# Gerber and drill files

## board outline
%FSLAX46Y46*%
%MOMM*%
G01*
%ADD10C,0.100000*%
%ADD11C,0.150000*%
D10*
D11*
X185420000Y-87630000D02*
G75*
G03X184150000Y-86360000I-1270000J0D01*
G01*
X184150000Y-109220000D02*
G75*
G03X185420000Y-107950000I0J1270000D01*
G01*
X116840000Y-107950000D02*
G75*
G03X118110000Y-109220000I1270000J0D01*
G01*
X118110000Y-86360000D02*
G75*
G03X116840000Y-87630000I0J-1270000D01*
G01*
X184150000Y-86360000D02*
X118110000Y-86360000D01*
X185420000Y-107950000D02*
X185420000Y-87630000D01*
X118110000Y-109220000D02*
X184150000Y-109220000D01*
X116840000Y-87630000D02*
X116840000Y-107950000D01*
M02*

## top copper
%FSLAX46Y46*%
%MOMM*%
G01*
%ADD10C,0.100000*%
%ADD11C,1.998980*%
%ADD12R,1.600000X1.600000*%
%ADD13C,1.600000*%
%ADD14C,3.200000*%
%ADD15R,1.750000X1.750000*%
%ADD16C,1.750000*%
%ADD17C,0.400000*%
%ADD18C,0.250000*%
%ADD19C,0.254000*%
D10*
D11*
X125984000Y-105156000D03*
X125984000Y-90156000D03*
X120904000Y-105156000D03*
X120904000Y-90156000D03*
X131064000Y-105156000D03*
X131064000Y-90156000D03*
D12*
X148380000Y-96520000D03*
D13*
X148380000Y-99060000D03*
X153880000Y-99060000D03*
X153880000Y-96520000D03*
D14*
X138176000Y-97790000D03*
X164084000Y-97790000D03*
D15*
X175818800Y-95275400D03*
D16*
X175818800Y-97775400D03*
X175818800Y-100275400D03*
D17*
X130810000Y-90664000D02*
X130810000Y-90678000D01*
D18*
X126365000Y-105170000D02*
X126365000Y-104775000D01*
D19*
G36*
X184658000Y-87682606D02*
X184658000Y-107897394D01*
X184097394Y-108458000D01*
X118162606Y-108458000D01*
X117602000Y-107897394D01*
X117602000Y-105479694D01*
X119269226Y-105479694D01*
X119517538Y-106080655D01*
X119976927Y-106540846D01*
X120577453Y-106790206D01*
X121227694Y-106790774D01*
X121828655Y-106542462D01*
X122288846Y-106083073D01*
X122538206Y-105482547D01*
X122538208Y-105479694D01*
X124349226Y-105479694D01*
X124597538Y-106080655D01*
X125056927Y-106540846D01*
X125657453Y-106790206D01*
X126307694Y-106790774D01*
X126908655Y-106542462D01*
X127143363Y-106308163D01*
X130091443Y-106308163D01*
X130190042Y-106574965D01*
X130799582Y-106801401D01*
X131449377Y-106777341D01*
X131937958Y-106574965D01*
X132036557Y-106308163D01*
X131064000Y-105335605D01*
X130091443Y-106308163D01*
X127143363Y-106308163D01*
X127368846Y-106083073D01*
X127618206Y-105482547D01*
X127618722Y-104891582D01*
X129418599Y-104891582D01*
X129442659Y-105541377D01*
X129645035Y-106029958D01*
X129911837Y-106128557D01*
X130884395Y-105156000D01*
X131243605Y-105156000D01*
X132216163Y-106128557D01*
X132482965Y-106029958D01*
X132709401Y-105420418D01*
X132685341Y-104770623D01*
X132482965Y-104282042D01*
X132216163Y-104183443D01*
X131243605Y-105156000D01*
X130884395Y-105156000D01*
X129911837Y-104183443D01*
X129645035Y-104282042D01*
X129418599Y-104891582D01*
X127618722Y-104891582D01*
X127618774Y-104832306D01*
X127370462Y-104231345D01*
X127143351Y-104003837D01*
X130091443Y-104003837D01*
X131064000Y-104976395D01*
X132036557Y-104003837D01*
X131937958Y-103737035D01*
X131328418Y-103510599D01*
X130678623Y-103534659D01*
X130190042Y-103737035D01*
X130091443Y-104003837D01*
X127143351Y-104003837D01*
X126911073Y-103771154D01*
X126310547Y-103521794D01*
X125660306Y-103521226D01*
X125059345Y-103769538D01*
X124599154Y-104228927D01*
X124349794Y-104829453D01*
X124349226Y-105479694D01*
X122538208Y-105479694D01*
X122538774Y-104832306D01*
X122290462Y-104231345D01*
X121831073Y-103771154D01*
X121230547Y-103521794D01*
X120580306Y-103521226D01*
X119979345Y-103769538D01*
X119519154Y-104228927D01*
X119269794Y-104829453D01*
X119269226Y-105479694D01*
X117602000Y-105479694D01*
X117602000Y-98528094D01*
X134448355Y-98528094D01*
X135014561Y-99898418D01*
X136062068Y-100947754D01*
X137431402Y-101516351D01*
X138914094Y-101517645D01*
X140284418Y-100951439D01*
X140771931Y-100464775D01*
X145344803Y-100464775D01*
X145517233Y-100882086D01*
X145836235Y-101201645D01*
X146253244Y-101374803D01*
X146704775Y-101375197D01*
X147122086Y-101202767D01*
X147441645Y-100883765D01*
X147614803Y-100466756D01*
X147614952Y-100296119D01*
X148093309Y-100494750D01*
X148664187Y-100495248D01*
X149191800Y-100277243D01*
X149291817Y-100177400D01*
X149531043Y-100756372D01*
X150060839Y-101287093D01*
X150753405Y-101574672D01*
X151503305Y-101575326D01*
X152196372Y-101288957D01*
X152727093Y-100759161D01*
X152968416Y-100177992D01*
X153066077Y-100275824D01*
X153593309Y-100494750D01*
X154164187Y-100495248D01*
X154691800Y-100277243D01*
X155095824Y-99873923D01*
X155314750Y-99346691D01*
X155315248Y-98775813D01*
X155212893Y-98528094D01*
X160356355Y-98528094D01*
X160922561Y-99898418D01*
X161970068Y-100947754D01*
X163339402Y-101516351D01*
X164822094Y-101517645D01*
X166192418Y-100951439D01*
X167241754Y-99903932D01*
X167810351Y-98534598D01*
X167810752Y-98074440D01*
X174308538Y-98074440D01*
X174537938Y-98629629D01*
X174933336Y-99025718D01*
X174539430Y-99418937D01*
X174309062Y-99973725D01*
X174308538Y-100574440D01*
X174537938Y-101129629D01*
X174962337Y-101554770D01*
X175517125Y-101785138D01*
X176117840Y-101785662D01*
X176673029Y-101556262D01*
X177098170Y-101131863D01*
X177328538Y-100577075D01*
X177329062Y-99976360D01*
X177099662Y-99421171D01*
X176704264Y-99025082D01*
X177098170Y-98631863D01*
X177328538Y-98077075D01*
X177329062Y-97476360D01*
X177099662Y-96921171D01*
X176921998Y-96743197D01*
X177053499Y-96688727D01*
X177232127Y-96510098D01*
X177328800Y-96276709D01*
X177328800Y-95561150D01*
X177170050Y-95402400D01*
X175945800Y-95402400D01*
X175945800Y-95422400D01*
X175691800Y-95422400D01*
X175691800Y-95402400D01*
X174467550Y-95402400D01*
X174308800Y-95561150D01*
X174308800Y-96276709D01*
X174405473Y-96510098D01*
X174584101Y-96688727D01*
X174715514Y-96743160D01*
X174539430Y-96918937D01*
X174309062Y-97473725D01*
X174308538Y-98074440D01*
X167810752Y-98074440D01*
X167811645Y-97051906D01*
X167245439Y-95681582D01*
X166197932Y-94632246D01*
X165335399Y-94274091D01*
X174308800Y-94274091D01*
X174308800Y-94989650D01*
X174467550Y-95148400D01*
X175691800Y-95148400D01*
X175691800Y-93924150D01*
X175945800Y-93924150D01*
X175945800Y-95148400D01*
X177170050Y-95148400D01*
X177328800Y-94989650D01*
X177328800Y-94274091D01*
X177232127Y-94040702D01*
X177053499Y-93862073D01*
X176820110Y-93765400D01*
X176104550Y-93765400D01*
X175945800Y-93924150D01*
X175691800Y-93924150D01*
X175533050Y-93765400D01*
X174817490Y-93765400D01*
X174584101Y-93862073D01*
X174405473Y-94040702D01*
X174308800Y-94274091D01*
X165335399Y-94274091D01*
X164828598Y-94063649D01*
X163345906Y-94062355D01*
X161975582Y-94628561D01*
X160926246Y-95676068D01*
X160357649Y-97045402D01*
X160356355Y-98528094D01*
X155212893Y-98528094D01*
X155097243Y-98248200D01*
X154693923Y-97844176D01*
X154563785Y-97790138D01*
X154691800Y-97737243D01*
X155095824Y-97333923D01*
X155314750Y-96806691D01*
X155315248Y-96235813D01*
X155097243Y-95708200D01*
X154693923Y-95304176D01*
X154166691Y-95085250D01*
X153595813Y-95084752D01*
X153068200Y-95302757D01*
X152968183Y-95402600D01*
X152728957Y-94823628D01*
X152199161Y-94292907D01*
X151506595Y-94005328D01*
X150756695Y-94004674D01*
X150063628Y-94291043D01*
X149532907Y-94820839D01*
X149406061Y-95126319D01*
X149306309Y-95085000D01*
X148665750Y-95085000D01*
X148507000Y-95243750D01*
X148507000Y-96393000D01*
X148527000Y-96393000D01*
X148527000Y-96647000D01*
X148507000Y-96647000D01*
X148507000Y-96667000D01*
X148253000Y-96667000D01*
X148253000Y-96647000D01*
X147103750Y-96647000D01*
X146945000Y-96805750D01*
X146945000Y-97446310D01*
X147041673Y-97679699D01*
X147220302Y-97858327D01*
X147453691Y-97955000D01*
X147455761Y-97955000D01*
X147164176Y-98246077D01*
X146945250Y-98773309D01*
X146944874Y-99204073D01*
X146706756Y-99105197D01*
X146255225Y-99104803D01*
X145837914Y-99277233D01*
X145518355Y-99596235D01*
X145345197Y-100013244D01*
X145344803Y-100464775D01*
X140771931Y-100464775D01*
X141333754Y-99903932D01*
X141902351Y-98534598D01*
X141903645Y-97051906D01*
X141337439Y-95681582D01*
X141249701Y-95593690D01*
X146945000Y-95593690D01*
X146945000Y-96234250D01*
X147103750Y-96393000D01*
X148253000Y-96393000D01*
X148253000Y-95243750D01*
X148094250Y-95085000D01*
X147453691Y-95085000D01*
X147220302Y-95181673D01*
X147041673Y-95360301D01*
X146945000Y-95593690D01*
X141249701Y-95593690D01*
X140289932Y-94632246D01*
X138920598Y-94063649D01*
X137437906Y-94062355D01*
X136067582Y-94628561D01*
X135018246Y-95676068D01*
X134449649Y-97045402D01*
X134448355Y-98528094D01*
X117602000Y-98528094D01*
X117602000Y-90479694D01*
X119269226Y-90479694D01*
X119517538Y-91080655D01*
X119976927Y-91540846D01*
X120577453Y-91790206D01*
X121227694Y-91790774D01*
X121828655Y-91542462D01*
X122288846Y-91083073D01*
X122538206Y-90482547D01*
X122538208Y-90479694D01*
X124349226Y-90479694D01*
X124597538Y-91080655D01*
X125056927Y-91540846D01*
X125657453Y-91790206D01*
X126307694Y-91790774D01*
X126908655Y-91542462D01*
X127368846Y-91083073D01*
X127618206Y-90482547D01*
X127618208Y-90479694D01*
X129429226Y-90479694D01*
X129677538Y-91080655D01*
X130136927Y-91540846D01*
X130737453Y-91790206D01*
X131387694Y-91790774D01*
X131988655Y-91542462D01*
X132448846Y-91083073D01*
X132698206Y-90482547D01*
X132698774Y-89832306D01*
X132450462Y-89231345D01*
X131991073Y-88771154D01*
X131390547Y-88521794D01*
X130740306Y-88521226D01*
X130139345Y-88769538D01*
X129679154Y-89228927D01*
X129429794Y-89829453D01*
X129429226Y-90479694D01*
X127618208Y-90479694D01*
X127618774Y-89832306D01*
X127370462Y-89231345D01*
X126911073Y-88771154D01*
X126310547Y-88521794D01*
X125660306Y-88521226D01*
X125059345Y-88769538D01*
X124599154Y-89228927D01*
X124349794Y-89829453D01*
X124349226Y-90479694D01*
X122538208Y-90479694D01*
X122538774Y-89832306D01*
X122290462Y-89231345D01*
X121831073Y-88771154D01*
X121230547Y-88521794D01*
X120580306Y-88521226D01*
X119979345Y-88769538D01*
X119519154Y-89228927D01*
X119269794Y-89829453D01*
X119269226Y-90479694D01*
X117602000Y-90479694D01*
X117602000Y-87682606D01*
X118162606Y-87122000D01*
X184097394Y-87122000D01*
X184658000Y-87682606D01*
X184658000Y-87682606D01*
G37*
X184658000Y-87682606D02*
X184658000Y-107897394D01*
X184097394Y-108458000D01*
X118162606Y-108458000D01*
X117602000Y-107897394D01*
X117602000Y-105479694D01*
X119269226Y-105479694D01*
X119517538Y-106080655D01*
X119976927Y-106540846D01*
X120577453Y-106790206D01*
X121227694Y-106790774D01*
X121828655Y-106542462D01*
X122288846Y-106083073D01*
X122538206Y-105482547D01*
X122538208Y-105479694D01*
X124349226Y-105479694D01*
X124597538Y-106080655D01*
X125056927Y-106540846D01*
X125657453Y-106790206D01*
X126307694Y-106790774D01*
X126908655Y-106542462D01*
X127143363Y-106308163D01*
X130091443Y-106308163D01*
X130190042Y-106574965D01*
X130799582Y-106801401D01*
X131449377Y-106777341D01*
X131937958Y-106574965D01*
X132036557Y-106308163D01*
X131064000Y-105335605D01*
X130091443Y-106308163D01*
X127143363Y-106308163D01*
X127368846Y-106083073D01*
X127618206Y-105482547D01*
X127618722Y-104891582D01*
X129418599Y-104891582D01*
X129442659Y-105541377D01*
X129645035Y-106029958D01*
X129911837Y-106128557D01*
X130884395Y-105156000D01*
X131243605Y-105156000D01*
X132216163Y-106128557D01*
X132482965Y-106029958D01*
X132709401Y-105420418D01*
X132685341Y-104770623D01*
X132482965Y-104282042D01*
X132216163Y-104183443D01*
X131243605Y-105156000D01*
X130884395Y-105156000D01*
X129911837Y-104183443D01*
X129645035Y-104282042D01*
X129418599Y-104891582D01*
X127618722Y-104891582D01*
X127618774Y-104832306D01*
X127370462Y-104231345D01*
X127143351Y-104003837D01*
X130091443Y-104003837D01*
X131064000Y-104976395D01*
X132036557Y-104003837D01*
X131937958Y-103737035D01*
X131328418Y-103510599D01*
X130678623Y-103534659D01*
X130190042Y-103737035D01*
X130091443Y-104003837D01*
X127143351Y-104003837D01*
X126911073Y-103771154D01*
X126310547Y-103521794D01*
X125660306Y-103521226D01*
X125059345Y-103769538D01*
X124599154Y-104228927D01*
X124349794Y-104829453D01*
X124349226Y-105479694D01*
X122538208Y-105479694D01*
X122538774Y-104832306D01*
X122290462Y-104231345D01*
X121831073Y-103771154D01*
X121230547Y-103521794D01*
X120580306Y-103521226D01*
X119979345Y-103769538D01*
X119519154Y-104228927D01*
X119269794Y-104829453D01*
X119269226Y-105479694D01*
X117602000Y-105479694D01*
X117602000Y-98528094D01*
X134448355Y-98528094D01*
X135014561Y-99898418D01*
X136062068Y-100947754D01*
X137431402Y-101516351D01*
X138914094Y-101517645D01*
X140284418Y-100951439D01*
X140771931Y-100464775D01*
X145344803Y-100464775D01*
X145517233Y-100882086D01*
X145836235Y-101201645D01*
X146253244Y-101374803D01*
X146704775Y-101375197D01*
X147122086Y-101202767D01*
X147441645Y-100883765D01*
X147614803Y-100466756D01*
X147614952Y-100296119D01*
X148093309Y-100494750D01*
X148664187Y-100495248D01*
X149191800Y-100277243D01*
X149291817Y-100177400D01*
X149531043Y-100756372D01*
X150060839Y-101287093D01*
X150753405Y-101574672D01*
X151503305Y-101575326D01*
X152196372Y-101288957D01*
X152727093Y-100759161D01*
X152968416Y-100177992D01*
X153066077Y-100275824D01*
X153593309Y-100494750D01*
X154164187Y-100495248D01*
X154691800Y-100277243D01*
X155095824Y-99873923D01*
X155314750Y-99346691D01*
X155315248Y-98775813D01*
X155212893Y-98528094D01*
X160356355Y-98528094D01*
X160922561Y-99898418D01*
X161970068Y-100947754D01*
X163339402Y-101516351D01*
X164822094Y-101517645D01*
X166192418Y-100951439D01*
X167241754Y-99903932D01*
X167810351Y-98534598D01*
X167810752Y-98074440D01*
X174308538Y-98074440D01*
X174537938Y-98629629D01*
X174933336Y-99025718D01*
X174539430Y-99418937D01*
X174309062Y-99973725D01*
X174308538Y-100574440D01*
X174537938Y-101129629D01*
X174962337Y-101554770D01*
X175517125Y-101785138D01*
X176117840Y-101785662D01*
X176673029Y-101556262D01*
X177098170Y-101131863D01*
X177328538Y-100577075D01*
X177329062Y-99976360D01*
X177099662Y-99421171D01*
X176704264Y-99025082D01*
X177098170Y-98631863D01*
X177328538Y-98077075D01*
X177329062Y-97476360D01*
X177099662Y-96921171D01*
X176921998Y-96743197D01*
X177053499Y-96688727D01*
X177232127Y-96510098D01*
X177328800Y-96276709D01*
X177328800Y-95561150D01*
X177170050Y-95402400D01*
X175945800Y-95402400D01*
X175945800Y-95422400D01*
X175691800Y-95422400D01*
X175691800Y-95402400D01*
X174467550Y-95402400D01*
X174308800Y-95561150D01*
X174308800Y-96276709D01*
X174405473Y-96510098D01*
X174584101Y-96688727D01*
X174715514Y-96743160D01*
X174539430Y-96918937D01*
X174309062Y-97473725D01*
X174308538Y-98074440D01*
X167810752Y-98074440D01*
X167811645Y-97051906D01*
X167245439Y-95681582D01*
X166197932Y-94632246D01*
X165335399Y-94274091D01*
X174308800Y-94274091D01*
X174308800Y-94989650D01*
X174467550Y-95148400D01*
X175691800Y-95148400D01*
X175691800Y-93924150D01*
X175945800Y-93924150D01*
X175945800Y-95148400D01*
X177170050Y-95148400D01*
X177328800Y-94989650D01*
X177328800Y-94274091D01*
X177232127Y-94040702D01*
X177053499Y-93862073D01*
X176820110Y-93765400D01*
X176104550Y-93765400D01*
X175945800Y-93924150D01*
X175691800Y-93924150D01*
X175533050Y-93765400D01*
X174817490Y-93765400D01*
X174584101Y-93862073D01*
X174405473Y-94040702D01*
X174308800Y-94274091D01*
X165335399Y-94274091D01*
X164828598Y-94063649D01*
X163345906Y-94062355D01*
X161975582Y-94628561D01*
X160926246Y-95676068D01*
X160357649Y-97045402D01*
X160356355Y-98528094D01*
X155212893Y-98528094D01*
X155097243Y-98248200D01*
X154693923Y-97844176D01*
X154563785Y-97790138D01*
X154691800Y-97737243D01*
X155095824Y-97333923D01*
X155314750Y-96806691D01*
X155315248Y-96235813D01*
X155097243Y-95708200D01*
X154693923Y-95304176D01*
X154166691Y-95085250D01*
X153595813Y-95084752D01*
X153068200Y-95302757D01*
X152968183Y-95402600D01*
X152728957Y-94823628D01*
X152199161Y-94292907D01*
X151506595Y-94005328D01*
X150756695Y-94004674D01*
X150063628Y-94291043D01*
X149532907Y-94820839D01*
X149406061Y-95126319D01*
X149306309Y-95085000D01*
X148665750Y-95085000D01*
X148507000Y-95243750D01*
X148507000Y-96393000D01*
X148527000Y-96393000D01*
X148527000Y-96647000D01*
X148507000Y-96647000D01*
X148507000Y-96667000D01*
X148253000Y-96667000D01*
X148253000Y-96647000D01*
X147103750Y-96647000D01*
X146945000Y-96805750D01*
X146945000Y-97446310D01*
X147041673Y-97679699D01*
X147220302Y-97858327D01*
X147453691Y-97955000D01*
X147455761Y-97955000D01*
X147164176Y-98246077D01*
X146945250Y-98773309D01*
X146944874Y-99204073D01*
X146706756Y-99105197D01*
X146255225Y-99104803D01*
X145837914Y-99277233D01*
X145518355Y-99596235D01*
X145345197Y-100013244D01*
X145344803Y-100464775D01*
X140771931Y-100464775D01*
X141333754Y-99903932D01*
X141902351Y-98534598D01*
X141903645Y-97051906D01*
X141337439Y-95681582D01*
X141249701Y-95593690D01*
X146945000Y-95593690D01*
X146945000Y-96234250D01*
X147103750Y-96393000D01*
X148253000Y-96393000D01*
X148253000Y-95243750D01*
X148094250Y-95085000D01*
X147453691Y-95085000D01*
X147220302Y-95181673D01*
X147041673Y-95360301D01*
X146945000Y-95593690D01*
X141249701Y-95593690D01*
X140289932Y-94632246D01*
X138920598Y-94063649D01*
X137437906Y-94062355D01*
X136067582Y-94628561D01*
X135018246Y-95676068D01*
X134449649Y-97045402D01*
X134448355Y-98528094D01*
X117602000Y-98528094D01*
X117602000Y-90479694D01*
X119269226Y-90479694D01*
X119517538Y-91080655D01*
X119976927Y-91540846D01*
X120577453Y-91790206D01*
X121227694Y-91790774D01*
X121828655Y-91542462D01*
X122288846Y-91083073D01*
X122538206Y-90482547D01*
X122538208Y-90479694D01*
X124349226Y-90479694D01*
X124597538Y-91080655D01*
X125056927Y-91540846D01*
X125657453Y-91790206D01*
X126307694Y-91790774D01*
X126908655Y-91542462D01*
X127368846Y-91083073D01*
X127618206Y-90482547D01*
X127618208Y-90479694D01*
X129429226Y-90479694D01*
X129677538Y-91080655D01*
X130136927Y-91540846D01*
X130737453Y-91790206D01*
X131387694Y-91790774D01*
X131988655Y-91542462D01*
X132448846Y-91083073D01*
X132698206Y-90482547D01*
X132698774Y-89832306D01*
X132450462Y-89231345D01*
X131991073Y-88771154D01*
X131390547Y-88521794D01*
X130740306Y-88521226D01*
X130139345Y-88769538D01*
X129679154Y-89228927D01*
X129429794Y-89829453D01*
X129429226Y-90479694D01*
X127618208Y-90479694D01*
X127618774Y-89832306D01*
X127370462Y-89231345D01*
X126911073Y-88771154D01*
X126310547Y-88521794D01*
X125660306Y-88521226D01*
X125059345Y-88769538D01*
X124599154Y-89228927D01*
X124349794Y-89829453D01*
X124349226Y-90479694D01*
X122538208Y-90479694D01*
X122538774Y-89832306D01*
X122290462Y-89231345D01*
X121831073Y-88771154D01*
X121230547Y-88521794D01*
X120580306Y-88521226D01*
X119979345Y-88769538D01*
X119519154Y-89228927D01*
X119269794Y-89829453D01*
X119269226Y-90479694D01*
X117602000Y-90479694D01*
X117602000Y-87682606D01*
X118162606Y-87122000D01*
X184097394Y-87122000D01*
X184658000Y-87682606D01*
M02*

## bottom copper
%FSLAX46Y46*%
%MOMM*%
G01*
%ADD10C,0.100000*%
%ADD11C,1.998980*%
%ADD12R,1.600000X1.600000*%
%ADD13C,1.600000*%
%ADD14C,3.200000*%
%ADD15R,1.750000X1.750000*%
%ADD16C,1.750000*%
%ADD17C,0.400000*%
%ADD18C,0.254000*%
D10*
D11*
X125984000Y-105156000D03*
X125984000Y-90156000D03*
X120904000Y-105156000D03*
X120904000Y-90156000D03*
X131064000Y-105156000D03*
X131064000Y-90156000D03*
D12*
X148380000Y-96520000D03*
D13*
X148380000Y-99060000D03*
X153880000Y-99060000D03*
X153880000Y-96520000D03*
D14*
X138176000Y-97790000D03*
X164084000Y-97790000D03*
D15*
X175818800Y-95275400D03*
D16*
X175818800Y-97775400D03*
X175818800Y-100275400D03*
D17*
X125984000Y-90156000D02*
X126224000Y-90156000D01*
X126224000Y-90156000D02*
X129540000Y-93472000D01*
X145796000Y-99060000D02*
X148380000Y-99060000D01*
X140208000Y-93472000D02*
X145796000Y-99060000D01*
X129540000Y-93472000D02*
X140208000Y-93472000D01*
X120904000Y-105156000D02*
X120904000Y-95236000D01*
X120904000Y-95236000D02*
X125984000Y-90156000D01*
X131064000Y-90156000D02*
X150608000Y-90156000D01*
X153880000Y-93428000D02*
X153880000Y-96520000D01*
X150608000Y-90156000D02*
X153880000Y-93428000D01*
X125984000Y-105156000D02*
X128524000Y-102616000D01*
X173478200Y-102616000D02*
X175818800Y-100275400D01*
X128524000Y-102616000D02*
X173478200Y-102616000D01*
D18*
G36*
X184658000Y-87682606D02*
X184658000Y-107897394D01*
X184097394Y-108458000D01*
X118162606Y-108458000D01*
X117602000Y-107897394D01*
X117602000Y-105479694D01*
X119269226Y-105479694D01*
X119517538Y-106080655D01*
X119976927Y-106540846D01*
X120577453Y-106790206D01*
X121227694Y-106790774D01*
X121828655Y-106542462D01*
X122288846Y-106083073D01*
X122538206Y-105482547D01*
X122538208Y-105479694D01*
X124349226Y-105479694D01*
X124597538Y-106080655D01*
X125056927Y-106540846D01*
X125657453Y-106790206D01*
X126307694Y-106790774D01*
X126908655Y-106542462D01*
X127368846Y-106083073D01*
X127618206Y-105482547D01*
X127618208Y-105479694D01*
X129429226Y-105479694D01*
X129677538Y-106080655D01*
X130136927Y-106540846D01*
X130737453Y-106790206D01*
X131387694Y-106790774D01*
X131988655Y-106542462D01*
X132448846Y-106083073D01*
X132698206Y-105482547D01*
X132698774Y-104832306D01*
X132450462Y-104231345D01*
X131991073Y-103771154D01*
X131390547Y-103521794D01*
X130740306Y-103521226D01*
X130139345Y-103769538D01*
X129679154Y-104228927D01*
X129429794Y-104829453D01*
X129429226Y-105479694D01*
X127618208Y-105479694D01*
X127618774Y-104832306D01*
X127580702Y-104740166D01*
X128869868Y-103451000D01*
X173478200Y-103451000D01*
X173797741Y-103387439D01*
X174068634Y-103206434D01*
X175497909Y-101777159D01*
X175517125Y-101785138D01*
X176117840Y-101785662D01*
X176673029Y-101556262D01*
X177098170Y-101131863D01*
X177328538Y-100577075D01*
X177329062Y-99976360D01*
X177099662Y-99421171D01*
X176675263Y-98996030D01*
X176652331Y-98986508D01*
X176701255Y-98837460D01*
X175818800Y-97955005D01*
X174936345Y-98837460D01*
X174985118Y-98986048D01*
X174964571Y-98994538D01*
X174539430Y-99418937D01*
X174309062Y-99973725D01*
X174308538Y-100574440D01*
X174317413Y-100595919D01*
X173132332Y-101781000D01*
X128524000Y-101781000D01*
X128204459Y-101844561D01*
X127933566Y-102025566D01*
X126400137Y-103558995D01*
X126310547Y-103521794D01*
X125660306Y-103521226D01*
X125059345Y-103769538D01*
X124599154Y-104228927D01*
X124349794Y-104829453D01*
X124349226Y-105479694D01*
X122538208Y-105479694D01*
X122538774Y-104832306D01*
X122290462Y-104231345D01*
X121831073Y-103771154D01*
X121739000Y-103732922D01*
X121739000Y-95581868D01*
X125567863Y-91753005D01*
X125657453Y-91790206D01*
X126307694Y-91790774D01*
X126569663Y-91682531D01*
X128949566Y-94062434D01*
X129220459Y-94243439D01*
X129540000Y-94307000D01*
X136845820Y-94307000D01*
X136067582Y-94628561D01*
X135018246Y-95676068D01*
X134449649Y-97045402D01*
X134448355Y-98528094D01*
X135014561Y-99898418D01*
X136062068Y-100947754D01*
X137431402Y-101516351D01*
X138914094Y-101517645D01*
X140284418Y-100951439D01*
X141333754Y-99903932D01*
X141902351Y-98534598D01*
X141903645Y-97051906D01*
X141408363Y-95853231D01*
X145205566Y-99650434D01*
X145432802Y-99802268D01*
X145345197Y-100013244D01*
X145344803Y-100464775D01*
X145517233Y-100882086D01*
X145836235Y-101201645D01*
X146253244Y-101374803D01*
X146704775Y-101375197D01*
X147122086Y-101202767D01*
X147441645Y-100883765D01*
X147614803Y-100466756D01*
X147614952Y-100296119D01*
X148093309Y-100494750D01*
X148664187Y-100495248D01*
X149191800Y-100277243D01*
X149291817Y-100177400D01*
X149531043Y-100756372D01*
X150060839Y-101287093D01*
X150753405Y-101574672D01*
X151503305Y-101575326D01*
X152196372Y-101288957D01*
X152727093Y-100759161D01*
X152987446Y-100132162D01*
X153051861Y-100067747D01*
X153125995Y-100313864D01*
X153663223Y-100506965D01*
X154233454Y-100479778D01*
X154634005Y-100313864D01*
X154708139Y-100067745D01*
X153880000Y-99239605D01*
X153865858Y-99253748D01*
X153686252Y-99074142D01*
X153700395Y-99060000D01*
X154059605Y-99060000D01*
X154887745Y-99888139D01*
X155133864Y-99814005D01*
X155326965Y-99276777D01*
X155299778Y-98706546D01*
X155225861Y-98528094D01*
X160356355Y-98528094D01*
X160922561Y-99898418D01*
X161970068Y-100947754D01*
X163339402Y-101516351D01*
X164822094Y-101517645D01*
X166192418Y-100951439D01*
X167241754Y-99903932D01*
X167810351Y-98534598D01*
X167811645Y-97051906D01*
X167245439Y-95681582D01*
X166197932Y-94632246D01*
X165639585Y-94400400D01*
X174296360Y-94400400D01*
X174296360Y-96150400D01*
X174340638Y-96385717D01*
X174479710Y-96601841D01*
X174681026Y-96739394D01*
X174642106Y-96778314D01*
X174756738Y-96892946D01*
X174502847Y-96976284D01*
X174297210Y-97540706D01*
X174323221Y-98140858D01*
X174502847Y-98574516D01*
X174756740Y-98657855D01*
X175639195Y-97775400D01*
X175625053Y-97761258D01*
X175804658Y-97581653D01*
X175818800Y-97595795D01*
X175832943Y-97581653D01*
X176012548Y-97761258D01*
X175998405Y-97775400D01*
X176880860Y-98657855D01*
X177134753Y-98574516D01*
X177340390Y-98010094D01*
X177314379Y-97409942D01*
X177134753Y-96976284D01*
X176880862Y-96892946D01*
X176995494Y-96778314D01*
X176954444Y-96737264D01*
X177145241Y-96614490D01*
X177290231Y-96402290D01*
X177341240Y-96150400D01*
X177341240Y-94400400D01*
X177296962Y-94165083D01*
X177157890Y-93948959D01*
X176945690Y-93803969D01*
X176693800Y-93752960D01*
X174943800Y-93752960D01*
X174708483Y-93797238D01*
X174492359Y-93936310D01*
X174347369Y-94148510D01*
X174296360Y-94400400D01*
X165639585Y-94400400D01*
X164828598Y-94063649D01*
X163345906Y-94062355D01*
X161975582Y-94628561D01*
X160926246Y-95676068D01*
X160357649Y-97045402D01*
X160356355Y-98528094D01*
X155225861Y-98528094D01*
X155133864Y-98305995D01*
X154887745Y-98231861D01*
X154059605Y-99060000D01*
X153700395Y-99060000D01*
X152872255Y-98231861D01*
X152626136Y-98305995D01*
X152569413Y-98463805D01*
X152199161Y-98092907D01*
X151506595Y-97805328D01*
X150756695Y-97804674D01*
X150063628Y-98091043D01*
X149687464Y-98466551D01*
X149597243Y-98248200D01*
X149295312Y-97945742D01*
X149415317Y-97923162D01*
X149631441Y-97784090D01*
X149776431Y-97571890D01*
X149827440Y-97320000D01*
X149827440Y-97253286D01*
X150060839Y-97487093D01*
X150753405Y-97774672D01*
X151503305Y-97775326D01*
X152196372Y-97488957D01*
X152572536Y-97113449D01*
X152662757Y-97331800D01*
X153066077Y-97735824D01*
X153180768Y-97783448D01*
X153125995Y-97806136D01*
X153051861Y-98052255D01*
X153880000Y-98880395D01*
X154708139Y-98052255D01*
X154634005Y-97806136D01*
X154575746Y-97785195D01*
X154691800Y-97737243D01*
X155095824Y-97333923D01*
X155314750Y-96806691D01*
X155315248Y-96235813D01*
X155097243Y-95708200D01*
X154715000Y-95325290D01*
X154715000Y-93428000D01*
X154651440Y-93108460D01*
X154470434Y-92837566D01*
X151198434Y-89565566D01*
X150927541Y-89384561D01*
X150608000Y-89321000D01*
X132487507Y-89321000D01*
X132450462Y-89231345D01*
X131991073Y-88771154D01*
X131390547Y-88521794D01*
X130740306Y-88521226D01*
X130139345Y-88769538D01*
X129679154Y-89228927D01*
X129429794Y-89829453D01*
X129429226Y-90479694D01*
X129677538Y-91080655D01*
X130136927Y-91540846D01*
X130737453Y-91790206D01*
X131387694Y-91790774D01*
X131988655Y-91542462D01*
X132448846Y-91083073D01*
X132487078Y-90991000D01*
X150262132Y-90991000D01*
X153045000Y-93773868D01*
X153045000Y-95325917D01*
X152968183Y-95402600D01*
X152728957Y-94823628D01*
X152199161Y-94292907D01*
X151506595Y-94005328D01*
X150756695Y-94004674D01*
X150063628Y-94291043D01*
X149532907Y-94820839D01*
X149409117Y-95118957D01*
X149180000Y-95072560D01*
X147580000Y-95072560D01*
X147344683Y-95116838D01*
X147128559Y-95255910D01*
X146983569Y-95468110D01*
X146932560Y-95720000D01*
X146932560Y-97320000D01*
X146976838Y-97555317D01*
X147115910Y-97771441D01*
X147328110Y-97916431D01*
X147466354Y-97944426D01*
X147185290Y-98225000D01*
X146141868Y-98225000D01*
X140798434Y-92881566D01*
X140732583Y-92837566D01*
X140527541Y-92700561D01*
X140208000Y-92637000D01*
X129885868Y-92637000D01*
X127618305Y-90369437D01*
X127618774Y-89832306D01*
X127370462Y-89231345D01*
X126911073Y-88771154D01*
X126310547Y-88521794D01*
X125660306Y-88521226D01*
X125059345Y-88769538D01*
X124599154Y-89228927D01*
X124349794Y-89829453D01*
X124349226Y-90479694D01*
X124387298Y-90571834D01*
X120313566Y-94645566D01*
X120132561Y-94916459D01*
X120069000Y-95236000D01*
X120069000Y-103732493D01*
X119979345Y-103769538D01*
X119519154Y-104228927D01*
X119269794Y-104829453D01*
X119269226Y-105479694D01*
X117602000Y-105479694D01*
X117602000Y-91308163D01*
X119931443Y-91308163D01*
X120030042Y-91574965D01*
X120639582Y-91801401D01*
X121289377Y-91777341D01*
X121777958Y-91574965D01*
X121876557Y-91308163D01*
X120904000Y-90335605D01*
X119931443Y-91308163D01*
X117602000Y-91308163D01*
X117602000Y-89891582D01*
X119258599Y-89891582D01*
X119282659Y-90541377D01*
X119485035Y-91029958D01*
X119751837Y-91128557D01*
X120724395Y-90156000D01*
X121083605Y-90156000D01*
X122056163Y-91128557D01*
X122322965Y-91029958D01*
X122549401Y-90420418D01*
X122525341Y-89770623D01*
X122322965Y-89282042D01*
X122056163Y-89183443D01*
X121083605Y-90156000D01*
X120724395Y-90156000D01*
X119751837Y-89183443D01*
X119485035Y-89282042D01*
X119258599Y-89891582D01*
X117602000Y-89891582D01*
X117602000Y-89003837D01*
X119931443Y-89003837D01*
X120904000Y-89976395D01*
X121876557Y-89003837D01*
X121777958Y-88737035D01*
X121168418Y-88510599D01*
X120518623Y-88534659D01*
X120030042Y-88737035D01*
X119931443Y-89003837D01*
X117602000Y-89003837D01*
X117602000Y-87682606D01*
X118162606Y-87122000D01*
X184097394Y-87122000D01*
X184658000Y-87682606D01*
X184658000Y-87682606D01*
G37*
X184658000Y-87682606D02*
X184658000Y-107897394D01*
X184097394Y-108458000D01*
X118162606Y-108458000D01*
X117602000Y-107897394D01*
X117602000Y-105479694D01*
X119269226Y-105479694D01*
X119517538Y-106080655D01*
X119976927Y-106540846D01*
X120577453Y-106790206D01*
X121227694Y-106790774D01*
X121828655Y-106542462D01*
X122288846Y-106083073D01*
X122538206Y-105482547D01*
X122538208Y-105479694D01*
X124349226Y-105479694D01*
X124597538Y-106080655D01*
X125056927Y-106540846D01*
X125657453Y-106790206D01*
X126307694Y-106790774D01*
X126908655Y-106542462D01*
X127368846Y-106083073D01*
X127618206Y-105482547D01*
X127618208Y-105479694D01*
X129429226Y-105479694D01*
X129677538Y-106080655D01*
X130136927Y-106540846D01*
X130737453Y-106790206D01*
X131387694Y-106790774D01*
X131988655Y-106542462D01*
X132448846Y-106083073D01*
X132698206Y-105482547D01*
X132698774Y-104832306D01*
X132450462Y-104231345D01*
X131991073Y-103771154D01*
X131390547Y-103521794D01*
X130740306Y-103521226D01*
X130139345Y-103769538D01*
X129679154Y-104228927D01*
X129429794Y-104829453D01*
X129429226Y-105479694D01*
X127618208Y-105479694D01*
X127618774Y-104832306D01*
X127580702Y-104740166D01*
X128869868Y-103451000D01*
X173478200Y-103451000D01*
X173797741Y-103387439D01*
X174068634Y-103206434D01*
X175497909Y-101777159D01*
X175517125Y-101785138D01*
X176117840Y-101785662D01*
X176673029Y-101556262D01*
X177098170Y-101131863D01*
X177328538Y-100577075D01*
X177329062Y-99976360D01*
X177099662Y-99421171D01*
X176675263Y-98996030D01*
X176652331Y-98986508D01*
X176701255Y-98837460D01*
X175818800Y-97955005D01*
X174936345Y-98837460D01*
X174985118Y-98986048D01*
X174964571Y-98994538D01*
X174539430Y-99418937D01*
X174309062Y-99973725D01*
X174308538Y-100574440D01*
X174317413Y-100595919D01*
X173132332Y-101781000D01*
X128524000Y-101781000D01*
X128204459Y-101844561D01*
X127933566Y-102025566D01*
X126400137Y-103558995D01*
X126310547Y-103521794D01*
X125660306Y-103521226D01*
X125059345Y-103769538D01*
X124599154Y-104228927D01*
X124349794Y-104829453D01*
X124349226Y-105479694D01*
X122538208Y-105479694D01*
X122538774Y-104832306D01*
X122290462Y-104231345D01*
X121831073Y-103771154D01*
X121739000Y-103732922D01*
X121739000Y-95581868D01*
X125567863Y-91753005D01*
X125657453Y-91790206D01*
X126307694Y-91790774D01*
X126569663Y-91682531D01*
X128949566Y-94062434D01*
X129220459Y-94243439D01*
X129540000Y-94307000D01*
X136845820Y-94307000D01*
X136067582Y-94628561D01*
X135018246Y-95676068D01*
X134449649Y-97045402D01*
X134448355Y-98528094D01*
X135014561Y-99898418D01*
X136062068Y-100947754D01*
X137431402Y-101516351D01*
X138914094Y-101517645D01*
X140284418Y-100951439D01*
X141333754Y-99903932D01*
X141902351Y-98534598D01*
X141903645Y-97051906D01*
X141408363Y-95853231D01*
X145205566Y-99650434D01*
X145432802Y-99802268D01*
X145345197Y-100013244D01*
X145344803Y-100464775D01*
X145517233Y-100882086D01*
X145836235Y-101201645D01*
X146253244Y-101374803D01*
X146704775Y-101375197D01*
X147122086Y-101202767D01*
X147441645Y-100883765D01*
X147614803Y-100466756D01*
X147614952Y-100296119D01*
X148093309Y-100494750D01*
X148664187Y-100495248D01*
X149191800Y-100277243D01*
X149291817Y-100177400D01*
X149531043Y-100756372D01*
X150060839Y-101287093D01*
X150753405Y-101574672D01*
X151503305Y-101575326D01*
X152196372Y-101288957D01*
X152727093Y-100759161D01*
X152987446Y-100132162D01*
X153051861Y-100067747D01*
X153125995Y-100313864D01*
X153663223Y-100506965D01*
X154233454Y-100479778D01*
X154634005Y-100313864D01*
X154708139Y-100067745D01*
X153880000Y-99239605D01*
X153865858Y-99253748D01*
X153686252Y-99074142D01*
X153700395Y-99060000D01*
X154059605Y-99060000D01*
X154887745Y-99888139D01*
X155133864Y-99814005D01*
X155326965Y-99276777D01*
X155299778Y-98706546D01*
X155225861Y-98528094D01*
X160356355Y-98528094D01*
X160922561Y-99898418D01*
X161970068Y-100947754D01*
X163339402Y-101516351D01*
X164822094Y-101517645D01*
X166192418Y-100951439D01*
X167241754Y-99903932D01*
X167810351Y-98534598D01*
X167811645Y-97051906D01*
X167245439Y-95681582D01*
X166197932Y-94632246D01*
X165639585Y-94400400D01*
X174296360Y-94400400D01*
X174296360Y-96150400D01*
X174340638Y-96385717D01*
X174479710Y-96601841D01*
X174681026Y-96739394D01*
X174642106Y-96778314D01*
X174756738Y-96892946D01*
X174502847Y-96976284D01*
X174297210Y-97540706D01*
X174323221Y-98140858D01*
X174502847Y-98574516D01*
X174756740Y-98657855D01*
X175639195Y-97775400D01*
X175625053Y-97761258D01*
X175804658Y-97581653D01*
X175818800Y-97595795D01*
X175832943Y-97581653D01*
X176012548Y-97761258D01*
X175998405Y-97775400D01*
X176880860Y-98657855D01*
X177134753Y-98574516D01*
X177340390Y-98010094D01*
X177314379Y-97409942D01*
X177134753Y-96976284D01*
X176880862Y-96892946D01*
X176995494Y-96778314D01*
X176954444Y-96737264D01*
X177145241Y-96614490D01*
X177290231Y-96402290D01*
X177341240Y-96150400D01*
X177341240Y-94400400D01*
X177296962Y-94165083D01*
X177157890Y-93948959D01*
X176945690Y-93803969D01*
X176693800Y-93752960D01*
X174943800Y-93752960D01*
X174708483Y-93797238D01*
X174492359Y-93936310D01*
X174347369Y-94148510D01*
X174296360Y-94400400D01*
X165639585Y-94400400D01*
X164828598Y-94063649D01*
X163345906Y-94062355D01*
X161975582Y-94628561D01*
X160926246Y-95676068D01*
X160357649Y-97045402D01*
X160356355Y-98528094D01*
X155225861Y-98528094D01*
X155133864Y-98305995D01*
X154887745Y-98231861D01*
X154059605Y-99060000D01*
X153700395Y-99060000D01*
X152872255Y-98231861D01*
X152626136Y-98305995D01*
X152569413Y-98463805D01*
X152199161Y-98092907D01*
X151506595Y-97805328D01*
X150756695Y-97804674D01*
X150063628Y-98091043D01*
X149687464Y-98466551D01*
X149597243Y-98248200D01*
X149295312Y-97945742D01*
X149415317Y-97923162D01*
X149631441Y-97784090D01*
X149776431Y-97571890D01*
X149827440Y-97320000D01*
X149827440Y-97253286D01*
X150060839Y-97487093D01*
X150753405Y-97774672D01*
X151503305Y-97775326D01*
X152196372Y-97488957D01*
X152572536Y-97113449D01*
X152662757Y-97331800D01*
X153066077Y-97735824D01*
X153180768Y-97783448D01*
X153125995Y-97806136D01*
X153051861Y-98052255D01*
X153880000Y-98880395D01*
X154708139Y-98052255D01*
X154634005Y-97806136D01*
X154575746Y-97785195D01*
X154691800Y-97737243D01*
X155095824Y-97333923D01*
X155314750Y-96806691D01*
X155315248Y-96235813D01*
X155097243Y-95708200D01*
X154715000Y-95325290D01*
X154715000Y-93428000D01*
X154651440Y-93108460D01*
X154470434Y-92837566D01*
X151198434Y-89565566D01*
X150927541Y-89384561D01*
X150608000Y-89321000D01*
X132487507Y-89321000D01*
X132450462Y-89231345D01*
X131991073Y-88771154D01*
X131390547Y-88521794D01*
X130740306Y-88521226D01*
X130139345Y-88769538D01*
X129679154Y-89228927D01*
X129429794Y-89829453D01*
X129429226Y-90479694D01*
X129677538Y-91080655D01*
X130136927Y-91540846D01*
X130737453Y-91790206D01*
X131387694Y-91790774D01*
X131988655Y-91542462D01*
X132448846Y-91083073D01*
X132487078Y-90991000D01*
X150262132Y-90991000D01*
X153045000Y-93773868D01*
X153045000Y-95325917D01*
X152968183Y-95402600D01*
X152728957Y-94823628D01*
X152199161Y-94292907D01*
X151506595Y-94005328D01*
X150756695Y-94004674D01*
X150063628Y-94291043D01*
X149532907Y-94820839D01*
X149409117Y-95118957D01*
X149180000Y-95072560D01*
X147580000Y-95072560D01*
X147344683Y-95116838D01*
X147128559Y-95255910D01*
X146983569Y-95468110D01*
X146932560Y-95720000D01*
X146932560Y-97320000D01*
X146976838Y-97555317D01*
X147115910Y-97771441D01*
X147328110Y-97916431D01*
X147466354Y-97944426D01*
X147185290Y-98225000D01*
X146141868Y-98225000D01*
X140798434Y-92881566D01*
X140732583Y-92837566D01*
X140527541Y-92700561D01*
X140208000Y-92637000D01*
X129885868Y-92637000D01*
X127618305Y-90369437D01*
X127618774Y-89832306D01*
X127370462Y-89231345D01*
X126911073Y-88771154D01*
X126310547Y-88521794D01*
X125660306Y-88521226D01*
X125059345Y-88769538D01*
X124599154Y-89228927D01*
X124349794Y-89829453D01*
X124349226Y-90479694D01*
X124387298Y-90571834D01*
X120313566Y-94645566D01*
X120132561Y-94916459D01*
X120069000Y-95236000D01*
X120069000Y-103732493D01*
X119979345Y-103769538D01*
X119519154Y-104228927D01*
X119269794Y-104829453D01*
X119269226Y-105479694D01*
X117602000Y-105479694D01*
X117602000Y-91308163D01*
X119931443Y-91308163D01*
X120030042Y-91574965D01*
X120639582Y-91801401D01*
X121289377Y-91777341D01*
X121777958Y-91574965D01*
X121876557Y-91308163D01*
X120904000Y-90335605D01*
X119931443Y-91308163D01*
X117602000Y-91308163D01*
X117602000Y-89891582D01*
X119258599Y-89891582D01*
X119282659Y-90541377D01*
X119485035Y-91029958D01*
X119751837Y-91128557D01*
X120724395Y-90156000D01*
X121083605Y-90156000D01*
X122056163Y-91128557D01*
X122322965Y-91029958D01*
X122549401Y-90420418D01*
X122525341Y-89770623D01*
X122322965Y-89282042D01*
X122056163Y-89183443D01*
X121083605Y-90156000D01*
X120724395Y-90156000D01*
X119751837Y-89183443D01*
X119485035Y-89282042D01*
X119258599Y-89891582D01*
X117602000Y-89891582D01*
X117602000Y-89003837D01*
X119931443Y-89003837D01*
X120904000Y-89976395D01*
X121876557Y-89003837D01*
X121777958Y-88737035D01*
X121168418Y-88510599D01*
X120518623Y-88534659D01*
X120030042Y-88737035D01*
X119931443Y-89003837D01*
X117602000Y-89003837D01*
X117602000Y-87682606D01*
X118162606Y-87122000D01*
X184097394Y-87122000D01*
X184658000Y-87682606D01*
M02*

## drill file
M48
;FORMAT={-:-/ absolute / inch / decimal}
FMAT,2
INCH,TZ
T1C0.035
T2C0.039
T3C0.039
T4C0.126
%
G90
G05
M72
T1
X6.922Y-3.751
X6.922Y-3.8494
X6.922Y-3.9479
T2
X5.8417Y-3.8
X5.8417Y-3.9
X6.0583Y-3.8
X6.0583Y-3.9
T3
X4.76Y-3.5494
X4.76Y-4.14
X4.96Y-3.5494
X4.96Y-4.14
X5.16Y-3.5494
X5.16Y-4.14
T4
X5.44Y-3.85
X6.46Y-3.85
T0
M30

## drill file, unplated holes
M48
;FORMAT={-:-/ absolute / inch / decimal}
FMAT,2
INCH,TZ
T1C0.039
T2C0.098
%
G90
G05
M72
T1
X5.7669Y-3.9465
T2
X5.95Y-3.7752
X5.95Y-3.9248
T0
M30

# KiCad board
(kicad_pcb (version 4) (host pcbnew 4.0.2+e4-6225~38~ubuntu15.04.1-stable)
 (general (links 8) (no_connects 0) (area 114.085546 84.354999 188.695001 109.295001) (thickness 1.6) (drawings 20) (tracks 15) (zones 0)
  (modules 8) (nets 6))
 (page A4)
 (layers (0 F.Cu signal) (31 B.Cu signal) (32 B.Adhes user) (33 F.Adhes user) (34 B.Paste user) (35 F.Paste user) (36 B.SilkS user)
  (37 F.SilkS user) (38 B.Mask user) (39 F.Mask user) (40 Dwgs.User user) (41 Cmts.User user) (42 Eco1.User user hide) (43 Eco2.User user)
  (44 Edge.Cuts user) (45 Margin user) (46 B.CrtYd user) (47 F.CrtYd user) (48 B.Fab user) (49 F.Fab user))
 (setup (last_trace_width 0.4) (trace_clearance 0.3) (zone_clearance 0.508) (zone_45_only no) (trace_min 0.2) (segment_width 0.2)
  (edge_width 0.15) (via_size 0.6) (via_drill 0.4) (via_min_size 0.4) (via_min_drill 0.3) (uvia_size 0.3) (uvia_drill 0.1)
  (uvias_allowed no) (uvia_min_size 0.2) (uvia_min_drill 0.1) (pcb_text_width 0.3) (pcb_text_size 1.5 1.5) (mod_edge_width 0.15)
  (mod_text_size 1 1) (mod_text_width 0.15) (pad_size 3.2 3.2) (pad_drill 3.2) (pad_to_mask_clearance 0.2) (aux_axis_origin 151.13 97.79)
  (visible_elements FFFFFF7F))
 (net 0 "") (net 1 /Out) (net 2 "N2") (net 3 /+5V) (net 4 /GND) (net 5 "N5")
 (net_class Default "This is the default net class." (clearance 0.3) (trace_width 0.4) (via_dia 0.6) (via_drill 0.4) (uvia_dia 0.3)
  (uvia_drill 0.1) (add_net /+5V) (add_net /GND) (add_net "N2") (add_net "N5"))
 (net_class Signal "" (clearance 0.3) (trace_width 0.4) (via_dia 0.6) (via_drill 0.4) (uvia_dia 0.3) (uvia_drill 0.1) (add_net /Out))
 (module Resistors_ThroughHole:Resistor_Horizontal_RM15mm (layer B.Cu) (at 125.984 105.156 90)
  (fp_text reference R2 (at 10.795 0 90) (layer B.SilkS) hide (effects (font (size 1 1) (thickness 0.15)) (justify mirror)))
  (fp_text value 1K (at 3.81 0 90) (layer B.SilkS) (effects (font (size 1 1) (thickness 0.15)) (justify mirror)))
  (pad 1 thru_hole circle (at 0 0 90) (size 1.99898 1.99898) (drill 1.00076) (layers *.Cu *.SilkS *.Mask) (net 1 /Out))
  (pad 2 thru_hole circle (at 15 0 90) (size 1.99898 1.99898) (drill 1.00076) (layers *.Cu *.SilkS *.Mask) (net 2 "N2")))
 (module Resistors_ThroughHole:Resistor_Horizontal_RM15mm (layer B.Cu) (at 120.904 105.156 90)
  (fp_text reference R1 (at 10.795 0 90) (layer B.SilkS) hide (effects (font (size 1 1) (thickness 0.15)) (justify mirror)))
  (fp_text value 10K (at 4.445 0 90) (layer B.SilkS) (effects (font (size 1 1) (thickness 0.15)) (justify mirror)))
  (pad 1 thru_hole circle (at 0 0 90) (size 1.99898 1.99898) (drill 1.00076) (layers *.Cu *.SilkS *.Mask) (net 2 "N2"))
  (pad 2 thru_hole circle (at 15 0 90) (size 1.99898 1.99898) (drill 1.00076) (layers *.Cu *.SilkS *.Mask) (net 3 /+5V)))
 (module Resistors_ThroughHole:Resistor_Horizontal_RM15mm (layer B.Cu) (at 131.064 105.156 90)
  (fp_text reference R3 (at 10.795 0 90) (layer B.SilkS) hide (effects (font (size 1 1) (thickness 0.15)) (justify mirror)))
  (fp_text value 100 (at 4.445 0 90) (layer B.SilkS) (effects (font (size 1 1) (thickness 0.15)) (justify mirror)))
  (pad 1 thru_hole circle (at 0 0 90) (size 1.99898 1.99898) (drill 1.00076) (layers *.Cu *.SilkS *.Mask) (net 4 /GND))
  (pad 2 thru_hole circle (at 15 0 90) (size 1.99898 1.99898) (drill 1.00076) (layers *.Cu *.SilkS *.Mask) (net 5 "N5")))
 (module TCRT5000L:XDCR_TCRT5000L (layer F.Cu) (at 151.13 97.79) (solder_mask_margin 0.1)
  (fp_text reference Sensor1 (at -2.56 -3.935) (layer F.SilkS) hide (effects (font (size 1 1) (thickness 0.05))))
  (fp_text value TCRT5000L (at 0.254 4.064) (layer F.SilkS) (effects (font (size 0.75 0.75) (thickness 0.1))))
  (pad 1 thru_hole rect (at -2.75 -1.27) (size 1.6 1.6) (drill 1) (layers *.Cu *.Mask F.SilkS) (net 4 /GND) (solder_mask_margin 0.2))
  (pad 2 thru_hole circle (at -2.75 1.27) (size 1.6 1.6) (drill 1) (layers *.Cu *.Mask F.SilkS) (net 2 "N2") (solder_mask_margin 0.2))
  (pad 3 thru_hole circle (at 2.75 1.27) (size 1.6 1.6) (drill 1) (layers *.Cu *.Mask F.SilkS) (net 3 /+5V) (solder_mask_margin 0.2))
  (pad 4 thru_hole circle (at 2.75 -1.27) (size 1.6 1.6) (drill 1) (layers *.Cu *.Mask F.SilkS) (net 5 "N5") (solder_mask_margin 0.2))
  (pad Hole np_thru_hole circle (at 0 -1.9) (size 2.5 2.5) (drill 2.5) (layers))
  (pad Hole np_thru_hole circle (at 0 1.9) (size 2.5 2.5) (drill 2.5) (layers))
  (pad Hole np_thru_hole circle (at -4.65 2.45) (size 1 1) (drill 1) (layers)))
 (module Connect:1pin (layer F.Cu) (at 138.176 97.79)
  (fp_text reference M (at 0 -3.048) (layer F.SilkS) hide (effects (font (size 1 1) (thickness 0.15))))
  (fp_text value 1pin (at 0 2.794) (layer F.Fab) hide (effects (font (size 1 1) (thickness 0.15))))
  (pad 1 thru_hole circle (at 0 0) (size 3.2 3.2) (drill 3.2) (layers *.Cu *.Mask F.SilkS) (clearance 2)))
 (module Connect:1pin (layer F.Cu) (at 164.084 97.79)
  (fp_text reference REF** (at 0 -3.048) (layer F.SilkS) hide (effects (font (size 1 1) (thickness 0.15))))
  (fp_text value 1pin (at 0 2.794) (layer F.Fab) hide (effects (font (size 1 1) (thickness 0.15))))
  (pad 1 thru_hole circle (at 0 0) (size 3.2 3.2) (drill 3.2) (layers *.Cu *.Mask F.SilkS) (clearance 2)))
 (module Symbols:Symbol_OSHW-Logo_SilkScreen (layer F.Cu) (at 125.984 97.028)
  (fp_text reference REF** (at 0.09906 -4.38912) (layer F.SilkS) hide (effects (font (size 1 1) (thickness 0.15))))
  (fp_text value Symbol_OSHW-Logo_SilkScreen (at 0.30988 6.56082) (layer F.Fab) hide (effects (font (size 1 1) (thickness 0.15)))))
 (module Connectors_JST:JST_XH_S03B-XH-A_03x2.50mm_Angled (layer B.Cu) (at 175.8188 95.2754 270)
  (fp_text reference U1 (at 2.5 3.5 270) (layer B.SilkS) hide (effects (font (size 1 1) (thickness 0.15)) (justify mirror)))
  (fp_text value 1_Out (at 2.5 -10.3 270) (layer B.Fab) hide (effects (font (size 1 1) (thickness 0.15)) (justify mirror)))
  (pad 1 thru_hole rect (at 0 0 270) (size 1.75 1.75) (drill 0.9) (layers *.Cu *.Mask B.SilkS) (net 4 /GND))
  (pad 2 thru_hole circle (at 2.5 0 270) (size 1.75 1.75) (drill 0.9) (layers *.Cu *.Mask B.SilkS) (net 3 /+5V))
  (pad 3 thru_hole circle (at 5 0 270) (size 1.75 1.75) (drill 0.9) (layers *.Cu *.Mask B.SilkS) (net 1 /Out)))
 (gr_arc (start 184.15 87.63) (end 184.15 86.36) (angle 90) (layer Edge.Cuts) (width 0.15))
 (gr_arc (start 184.15 107.95) (end 185.42 107.95) (angle 90) (layer Edge.Cuts) (width 0.15))
 (gr_arc (start 118.11 107.95) (end 118.11 109.22) (angle 90) (layer Edge.Cuts) (width 0.15))
 (gr_arc (start 118.11 87.63) (end 116.84 87.63) (angle 90) (layer Edge.Cuts) (width 0.15))
 (gr_line (start 184.15 86.36) (end 118.11 86.36) (angle 90) (layer Edge.Cuts) (width 0.15))
 (gr_line (start 185.42 107.95) (end 185.42 87.63) (angle 90) (layer Edge.Cuts) (width 0.15))
 (gr_line (start 118.11 109.22) (end 184.15 109.22) (angle 90) (layer Edge.Cuts) (width 0.15))
 (gr_line (start 116.84 87.63) (end 116.84 107.95) (angle 90) (layer Edge.Cuts) (width 0.15))
 (segment (start 125.984 90.156) (end 126.224 90.156) (width 0.4) (layer B.Cu) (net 2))
 (segment (start 126.224 90.156) (end 129.54 93.472) (width 0.4) (layer B.Cu) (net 2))
 (segment (start 145.796 99.06) (end 148.38 99.06) (width 0.4) (layer B.Cu) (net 2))
 (segment (start 140.208 93.472) (end 145.796 99.06) (width 0.4) (layer B.Cu) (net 2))
 (segment (start 129.54 93.472) (end 140.208 93.472) (width 0.4) (layer B.Cu) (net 2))
 (segment (start 120.904 105.156) (end 120.904 95.236) (width 0.4) (layer B.Cu) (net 2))
 (segment (start 120.904 95.236) (end 125.984 90.156) (width 0.4) (layer B.Cu) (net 2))
 (segment (start 131.064 90.156) (end 150.608 90.156) (width 0.4) (layer B.Cu) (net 5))
 (segment (start 153.88 93.428) (end 153.88 96.52) (width 0.4) (layer B.Cu) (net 5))
 (segment (start 150.608 90.156) (end 153.88 93.428) (width 0.4) (layer B.Cu) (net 5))
 (segment (start 130.81 90.664) (end 130.81 90.678) (width 0.4) (layer F.Cu) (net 5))
 (segment (start 125.984 105.156) (end 128.524 102.616) (width 0.4) (layer B.Cu) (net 1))
 (segment (start 173.4782 102.616) (end 175.8188 100.2754) (width 0.4) (layer B.Cu) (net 1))
 (segment (start 128.524 102.616) (end 173.4782 102.616) (width 0.4) (layer B.Cu) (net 1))
 (segment (start 126.365 105.17) (end 126.365 104.775) (width 0.25) (layer F.Cu) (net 1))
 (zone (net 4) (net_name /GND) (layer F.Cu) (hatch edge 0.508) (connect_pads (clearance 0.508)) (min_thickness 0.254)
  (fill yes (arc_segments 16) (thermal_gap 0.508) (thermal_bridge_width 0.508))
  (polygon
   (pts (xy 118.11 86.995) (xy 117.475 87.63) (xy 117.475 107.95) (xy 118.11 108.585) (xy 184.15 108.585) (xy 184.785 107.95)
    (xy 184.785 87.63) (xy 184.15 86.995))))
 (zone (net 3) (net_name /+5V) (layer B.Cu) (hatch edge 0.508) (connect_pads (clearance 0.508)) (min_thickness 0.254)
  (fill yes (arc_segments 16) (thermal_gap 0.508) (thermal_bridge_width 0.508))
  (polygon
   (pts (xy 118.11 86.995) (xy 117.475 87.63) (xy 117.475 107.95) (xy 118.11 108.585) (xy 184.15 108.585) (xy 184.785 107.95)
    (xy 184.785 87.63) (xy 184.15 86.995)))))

